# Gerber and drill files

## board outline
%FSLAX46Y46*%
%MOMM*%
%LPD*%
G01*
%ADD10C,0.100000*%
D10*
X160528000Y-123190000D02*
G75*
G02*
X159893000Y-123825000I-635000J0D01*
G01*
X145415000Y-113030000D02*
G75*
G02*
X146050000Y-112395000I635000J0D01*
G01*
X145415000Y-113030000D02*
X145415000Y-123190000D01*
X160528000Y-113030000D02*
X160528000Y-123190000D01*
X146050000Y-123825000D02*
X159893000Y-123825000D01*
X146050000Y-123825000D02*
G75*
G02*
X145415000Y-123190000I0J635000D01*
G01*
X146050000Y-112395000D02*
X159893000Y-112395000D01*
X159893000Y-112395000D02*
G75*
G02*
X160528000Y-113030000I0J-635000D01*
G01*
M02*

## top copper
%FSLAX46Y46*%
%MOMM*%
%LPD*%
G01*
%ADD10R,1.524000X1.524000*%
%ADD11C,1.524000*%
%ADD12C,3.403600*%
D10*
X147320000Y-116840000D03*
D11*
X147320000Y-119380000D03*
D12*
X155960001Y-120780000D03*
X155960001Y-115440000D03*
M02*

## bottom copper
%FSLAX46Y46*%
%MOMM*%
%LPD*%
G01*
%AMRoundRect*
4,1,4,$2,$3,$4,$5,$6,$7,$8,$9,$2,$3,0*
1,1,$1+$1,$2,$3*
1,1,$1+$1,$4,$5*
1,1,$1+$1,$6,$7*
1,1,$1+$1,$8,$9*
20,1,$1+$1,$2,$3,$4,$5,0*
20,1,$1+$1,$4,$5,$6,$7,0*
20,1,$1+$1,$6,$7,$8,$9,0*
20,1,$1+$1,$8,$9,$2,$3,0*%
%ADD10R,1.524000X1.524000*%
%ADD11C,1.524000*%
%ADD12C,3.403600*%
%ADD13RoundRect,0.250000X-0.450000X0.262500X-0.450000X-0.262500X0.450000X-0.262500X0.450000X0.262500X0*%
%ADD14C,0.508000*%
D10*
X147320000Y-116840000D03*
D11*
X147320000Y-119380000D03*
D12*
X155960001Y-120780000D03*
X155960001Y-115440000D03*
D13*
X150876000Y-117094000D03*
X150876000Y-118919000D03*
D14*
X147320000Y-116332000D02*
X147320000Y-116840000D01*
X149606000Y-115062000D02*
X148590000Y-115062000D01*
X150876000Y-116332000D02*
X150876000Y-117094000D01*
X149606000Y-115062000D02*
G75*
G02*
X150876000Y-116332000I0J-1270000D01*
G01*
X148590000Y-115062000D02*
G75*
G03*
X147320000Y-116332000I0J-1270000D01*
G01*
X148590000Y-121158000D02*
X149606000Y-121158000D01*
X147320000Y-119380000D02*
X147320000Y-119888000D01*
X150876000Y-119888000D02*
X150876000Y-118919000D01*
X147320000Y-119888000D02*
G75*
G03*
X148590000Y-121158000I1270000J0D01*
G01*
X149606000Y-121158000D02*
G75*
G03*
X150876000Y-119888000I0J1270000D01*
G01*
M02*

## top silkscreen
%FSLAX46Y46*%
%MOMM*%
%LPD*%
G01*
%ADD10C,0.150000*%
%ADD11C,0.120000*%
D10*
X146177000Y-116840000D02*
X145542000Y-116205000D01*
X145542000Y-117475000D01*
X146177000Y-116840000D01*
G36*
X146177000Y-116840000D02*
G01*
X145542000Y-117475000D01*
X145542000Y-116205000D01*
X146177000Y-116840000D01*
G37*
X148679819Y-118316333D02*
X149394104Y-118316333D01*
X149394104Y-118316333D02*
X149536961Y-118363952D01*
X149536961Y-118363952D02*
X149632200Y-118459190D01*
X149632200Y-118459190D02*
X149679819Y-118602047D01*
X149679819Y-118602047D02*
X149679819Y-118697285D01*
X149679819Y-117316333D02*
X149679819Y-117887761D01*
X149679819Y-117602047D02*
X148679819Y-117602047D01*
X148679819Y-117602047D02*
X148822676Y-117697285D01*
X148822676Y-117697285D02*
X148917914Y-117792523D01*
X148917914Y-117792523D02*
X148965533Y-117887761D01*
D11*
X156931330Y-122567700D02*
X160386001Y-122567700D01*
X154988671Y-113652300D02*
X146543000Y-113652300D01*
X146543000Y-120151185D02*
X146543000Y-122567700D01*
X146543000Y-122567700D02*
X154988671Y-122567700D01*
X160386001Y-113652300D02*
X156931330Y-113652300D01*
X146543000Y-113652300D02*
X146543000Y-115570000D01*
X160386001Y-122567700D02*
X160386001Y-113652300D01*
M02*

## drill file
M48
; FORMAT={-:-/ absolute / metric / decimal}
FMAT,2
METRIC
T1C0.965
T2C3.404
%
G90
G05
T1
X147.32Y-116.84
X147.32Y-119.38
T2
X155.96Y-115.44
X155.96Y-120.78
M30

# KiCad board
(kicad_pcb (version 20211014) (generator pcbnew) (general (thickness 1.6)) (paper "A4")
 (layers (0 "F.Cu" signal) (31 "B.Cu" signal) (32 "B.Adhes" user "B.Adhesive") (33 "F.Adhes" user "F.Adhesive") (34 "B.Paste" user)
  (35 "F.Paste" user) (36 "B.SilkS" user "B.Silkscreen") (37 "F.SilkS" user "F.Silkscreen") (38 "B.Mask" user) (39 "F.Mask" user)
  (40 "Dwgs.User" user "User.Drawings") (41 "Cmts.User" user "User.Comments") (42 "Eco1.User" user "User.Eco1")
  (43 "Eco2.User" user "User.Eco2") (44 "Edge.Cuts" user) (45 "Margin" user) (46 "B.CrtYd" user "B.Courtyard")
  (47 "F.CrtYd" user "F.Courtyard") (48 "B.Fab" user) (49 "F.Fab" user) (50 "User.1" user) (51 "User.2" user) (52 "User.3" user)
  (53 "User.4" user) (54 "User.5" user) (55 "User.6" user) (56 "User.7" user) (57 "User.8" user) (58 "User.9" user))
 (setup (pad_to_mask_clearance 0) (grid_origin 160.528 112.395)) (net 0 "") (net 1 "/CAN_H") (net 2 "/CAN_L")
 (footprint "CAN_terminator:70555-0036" (layer "F.Cu") (at 147.32 116.84 90)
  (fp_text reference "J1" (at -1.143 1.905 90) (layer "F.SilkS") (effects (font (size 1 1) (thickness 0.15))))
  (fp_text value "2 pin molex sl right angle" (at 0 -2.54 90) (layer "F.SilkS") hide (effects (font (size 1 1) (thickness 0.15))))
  (fp_line (start -5.7277 9.61133) (end -5.7277 13.066001) (layer "F.SilkS") (width 0.12))
  (fp_line (start 3.1877 7.668671) (end 3.1877 -0.777) (layer "F.SilkS") (width 0.12))
  (fp_line (start -3.311185 -0.777) (end -5.7277 -0.777) (layer "F.SilkS") (width 0.12))
  (fp_line (start -5.7277 -0.777) (end -5.7277 7.668671) (layer "F.SilkS") (width 0.12))
  (fp_line (start 3.1877 13.066001) (end 3.1877 9.61133) (layer "F.SilkS") (width 0.12))
  (fp_line (start 3.1877 -0.777) (end 1.27 -0.777) (layer "F.SilkS") (width 0.12))
  (fp_line (start -5.7277 13.066001) (end 3.1877 13.066001) (layer "F.SilkS") (width 0.12))
  (pad "1" thru_hole rect (at 0 0 90) (size 1.524 1.524) (drill 0.9652) (layers *.Cu *.Mask) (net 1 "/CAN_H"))
  (pad "2" thru_hole circle (at -2.54 0 90) (size 1.524 1.524) (drill 0.9652) (layers *.Cu *.Mask) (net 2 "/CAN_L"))
  (pad "3" thru_hole circle (at -3.94 8.640001 90) (size 3.4036 3.4036) (drill 3.4036) (layers *.Cu *.Mask))
  (pad "4" thru_hole circle (at 1.4 8.640001 90) (size 3.4036 3.4036) (drill 3.4036) (layers *.Cu *.Mask)))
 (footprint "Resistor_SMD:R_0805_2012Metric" (layer "B.Cu") (at 150.876 118.0065 -90)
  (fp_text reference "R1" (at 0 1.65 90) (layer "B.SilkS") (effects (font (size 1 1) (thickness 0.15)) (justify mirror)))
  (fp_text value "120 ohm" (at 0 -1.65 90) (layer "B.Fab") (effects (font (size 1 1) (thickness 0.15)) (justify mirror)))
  (pad "1" smd roundrect (at -0.9125 0 270) (size 1.025 1.4) (layers "B.Cu" "B.Paste" "B.Mask") (roundrect_rratio 0.243902439)
   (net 1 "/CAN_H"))
  (pad "2" smd roundrect (at 0.9125 0 270) (size 1.025 1.4) (layers "B.Cu" "B.Paste" "B.Mask") (roundrect_rratio 0.243902439)
   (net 2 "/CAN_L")))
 (gr_poly (pts (xy 146.177 116.84) (xy 145.542 116.205) (xy 145.542 117.475)) (layer "F.SilkS") (width 0.15) (fill solid))
 (gr_arc (start 160.528 123.19) (mid 160.342013 123.639013) (end 159.893 123.825) (layer "Edge.Cuts") (width 0.1))
 (gr_arc (start 145.415 113.03) (mid 145.600987 112.580987) (end 146.05 112.395) (layer "Edge.Cuts") (width 0.1))
 (gr_line (start 145.415 113.03) (end 145.415 123.19) (layer "Edge.Cuts") (width 0.1))
 (gr_line (start 160.528 113.03) (end 160.528 123.19) (layer "Edge.Cuts") (width 0.1))
 (gr_line (start 146.05 123.825) (end 159.893 123.825) (layer "Edge.Cuts") (width 0.1))
 (gr_arc (start 146.05 123.825) (mid 145.600987 123.639013) (end 145.415 123.19) (layer "Edge.Cuts") (width 0.1))
 (gr_line (start 146.05 112.395) (end 159.893 112.395) (layer "Edge.Cuts") (width 0.1))
 (gr_arc (start 159.893 112.395) (mid 160.342013 112.580987) (end 160.528 113.03) (layer "Edge.Cuts") (width 0.1))
 (segment (start 147.32 116.332) (end 147.32 116.84) (width 0.508) (layer "B.Cu") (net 1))
 (segment (start 149.606 115.062) (end 148.59 115.062) (width 0.508) (layer "B.Cu") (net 1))
 (segment (start 150.876 116.332) (end 150.876 117.094) (width 0.508) (layer "B.Cu") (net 1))
 (arc (start 149.606 115.062) (mid 150.504026 115.433974) (end 150.876 116.332) (width 0.508) (layer "B.Cu") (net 1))
 (arc (start 148.59 115.062) (mid 147.691974 115.433974) (end 147.32 116.332) (width 0.508) (layer "B.Cu") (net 1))
 (segment (start 148.59 121.158) (end 149.606 121.158) (width 0.508) (layer "B.Cu") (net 2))
 (segment (start 147.32 119.38) (end 147.32 119.888) (width 0.508) (layer "B.Cu") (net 2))
 (segment (start 150.876 119.888) (end 150.876 118.919) (width 0.508) (layer "B.Cu") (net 2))
 (arc (start 147.32 119.888) (mid 147.691974 120.786026) (end 148.59 121.158) (width 0.508) (layer "B.Cu") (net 2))
 (arc (start 149.606 121.158) (mid 150.504026 120.786026) (end 150.876 119.888) (width 0.508) (layer "B.Cu") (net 2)))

